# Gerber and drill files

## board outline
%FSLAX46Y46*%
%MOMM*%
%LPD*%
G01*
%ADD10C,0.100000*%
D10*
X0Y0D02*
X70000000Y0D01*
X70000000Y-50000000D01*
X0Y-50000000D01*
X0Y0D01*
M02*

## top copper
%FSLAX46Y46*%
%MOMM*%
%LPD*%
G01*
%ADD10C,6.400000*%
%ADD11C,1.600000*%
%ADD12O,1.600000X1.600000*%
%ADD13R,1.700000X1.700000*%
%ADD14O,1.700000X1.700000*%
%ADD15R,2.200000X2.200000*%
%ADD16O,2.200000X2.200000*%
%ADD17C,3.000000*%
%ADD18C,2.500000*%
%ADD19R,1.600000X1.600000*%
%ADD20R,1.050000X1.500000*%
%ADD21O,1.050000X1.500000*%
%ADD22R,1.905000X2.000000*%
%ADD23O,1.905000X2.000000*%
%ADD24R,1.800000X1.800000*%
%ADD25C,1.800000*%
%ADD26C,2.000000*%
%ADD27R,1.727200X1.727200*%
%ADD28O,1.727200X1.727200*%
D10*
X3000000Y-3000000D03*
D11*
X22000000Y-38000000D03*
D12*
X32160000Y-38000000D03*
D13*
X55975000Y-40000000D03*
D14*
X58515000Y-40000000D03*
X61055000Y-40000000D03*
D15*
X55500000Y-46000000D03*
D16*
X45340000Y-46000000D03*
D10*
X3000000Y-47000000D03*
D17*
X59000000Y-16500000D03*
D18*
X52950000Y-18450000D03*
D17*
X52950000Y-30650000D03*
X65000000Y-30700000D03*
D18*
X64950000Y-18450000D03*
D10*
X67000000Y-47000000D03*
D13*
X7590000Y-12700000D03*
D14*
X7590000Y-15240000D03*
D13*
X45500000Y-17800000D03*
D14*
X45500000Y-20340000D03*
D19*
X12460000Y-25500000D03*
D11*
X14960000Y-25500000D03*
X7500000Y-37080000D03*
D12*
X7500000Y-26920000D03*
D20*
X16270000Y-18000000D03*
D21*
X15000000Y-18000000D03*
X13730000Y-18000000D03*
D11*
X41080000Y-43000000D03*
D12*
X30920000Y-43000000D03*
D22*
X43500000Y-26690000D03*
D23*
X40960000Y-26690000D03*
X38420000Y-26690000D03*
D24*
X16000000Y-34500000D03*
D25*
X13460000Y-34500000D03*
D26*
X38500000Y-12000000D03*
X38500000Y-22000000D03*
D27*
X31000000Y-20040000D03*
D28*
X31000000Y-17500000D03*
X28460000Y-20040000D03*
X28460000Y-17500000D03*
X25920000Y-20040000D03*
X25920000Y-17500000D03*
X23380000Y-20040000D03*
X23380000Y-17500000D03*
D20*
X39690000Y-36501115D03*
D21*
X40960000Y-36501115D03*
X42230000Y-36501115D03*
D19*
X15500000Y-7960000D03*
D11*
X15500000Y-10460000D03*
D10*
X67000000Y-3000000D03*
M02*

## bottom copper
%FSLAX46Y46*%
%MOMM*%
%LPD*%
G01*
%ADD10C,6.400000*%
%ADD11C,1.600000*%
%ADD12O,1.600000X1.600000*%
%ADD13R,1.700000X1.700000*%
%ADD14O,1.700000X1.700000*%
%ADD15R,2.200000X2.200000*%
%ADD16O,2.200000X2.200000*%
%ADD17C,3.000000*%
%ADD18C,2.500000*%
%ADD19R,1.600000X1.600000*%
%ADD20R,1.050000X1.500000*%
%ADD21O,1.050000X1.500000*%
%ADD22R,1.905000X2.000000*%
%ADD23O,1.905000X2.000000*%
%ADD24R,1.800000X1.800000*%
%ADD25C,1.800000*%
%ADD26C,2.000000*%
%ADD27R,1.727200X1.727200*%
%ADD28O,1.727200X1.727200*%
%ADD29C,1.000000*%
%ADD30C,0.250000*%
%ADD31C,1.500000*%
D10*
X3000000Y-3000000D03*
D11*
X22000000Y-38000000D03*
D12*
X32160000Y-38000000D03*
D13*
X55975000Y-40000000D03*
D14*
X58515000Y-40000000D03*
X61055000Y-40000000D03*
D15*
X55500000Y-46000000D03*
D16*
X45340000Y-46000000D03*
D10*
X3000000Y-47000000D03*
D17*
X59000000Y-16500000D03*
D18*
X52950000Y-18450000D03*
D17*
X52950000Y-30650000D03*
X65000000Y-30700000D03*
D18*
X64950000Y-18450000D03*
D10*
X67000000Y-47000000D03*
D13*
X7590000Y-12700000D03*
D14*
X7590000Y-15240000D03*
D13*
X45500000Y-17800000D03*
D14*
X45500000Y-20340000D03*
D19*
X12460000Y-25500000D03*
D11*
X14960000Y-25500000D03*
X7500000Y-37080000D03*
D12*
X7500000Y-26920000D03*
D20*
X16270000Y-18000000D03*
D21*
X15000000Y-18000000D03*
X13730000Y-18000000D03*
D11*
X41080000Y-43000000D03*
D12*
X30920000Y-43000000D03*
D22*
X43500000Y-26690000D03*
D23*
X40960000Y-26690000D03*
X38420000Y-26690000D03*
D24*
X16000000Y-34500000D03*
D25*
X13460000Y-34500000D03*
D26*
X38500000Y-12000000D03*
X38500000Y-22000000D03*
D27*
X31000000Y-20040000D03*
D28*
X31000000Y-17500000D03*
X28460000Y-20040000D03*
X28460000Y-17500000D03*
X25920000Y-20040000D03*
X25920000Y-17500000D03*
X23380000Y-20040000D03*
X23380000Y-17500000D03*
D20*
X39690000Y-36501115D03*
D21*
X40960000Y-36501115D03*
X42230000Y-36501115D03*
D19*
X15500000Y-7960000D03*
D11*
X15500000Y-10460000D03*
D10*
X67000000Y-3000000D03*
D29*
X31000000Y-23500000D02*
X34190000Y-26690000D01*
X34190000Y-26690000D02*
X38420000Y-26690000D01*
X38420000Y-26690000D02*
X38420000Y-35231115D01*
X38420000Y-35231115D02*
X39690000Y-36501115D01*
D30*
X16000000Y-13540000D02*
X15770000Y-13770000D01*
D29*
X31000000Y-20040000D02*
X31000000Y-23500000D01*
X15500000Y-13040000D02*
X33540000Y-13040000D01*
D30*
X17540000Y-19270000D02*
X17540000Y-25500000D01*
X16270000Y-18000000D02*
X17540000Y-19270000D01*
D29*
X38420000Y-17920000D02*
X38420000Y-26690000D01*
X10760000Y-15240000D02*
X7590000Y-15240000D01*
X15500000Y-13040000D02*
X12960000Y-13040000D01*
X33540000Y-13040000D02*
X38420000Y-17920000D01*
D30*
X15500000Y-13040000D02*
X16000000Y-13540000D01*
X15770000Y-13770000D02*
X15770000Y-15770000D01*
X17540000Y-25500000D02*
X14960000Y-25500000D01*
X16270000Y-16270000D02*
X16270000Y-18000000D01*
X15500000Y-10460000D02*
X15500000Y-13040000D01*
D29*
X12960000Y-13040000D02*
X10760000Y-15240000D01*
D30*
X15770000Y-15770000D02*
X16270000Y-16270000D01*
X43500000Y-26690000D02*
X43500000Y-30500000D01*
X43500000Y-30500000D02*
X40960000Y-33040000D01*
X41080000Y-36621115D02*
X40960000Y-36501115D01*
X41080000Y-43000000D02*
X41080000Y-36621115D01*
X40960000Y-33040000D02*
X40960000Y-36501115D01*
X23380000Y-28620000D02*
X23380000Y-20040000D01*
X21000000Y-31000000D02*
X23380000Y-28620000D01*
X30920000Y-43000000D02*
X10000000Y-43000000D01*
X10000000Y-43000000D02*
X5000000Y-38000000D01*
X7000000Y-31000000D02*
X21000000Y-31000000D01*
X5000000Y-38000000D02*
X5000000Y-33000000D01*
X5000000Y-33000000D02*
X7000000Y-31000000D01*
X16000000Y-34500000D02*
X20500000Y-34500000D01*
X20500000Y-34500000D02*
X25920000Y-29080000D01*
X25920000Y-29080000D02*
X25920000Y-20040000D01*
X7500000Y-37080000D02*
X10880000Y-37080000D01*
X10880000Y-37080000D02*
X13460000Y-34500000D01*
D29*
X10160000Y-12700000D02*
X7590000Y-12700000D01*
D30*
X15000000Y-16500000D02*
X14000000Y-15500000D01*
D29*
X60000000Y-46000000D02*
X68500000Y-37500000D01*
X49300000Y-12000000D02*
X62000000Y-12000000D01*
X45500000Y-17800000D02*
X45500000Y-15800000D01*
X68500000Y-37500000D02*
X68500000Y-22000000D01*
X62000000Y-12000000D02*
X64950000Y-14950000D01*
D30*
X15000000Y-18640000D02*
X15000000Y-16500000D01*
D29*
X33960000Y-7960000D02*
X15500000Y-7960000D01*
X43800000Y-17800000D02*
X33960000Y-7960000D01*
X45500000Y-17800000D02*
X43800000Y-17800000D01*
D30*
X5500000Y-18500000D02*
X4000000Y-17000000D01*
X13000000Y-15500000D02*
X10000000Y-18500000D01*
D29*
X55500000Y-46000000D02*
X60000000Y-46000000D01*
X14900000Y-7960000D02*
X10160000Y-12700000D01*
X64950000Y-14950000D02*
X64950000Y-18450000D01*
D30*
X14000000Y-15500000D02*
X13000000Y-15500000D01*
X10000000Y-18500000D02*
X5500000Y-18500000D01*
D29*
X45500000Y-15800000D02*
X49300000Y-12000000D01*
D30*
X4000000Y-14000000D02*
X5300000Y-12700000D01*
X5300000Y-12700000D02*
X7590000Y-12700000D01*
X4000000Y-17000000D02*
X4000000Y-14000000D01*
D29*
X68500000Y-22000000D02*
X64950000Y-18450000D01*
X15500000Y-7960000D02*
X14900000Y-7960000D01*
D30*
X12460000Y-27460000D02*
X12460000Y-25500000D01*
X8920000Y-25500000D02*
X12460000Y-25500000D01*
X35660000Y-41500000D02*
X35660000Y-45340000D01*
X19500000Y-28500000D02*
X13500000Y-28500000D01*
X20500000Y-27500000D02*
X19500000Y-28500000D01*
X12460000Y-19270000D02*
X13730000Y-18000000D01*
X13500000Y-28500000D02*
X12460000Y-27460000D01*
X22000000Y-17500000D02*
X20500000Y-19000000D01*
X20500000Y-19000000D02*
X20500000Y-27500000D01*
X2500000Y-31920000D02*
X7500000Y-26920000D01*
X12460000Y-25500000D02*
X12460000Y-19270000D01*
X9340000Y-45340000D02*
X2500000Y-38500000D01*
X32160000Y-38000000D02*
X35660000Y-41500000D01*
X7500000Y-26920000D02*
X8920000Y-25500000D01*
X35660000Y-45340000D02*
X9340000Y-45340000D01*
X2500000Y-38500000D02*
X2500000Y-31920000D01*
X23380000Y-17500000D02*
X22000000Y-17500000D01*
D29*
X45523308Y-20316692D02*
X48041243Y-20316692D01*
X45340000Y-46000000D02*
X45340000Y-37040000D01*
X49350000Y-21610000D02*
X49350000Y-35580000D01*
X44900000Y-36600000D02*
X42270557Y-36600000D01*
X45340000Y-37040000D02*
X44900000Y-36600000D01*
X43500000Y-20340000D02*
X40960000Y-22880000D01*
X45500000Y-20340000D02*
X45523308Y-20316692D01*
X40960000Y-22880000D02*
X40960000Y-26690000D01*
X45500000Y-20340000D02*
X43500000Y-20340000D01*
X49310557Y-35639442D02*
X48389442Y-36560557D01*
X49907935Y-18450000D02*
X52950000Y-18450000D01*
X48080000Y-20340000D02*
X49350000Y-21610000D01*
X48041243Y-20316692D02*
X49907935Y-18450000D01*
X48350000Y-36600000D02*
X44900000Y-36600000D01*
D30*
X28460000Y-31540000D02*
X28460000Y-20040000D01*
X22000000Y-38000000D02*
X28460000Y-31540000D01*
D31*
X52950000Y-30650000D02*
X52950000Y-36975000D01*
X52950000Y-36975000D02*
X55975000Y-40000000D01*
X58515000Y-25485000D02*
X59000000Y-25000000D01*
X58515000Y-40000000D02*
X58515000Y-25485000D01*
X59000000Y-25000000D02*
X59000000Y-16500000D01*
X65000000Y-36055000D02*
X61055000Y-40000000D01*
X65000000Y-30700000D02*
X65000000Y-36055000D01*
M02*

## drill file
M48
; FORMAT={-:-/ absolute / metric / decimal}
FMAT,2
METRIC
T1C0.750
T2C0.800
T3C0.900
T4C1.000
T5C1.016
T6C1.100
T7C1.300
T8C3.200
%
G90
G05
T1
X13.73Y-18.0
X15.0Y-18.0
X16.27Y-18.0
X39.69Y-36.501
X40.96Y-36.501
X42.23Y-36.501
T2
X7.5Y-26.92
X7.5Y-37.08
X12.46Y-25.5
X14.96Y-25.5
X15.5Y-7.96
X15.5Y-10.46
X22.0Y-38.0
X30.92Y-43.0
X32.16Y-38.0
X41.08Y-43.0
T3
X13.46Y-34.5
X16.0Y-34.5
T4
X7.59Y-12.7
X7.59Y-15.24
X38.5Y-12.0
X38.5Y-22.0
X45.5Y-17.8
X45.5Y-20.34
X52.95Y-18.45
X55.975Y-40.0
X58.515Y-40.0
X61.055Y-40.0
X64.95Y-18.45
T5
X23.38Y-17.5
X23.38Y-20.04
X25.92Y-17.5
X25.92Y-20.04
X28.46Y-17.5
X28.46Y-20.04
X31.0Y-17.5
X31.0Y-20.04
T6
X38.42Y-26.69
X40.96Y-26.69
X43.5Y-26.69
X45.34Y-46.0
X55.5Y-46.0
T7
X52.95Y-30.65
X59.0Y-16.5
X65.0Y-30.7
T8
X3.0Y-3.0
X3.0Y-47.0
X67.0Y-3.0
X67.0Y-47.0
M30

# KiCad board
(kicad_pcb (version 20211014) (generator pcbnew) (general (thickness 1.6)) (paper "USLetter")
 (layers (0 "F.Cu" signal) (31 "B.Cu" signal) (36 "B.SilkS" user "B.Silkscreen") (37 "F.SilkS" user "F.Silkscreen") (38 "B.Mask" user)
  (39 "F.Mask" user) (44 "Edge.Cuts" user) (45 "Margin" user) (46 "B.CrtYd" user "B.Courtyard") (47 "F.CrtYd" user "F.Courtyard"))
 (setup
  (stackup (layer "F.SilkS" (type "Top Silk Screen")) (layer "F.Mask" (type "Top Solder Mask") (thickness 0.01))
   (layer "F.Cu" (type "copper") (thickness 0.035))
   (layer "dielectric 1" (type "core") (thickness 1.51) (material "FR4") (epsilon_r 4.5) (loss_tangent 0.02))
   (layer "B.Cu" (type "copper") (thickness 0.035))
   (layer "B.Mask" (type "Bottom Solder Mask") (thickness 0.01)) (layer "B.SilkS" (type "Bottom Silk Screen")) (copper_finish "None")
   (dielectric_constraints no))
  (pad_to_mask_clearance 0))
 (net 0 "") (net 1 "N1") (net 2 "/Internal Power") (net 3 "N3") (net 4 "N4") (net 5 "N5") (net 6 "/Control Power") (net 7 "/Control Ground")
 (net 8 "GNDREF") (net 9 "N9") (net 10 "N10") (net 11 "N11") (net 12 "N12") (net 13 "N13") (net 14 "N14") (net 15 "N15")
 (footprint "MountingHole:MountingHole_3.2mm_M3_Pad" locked (layer "F.Cu") (at 3 3)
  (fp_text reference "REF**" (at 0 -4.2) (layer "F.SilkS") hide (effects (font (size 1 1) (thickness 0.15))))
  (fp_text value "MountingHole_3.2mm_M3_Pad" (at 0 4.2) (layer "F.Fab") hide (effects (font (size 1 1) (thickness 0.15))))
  (pad "1" thru_hole circle locked (at 0 0) (size 6.4 6.4) (drill 3.2) (layers *.Cu *.Mask)))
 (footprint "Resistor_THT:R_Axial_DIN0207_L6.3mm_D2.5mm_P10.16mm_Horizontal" (layer "F.Cu") (at 22 38)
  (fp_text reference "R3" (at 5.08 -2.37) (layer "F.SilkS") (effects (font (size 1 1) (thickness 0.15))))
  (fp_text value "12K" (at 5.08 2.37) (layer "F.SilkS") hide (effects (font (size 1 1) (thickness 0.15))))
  (pad "1" thru_hole circle (at 0 0) (size 1.6 1.6) (drill 0.8) (layers *.Cu *.Mask) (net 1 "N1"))
  (pad "2" thru_hole oval (at 10.16 0) (size 1.6 1.6) (drill 0.8) (layers *.Cu *.Mask) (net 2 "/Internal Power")))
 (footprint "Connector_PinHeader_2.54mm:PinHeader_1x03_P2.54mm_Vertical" (layer "F.Cu") (at 55.975 40 90)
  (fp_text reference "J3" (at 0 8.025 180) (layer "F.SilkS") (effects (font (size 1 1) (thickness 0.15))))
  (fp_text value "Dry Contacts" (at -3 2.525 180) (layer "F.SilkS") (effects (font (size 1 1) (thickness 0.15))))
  (pad "1" thru_hole rect (at 0 0 90) (size 1.7 1.7) (drill 1) (layers *.Cu *.Mask) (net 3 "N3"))
  (pad "2" thru_hole oval (at 0 2.54 90) (size 1.7 1.7) (drill 1) (layers *.Cu *.Mask) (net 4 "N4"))
  (pad "3" thru_hole oval (at 0 5.08 90) (size 1.7 1.7) (drill 1) (layers *.Cu *.Mask) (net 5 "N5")))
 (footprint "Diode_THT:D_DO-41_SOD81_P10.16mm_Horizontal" (layer "F.Cu") (at 55.5 46 180)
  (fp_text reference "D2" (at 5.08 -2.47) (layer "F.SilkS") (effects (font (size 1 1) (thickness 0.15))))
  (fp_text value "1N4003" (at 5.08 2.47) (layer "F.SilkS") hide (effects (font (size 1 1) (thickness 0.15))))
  (pad "1" thru_hole rect (at 0 0 180) (size 2.2 2.2) (drill 1.1) (layers *.Cu *.Mask) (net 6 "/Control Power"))
  (pad "2" thru_hole oval (at 10.16 0 180) (size 2.2 2.2) (drill 1.1) (layers *.Cu *.Mask) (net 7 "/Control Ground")))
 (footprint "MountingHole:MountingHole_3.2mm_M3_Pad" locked (layer "F.Cu") (at 3 47)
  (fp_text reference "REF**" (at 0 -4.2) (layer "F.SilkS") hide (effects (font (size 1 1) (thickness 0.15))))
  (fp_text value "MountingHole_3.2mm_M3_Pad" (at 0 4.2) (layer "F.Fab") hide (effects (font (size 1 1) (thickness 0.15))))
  (pad "4" thru_hole circle locked (at 0 0) (size 6.4 6.4) (drill 3.2) (layers *.Cu *.Mask)))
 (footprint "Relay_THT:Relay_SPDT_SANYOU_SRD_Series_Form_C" (layer "F.Cu") (at 59 16.5 -90)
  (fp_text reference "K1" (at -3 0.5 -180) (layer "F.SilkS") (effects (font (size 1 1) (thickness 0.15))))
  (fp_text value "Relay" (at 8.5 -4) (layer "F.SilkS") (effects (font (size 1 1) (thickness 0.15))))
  (pad "1" thru_hole circle (at 0 0) (size 3 3) (drill 1.3) (layers *.Cu *.Mask) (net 4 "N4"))
  (pad "2" thru_hole circle (at 1.95 6.05) (size 2.5 2.5) (drill 1) (layers *.Cu *.Mask) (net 7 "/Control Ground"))
  (pad "3" thru_hole circle (at 14.15 6.05) (size 3 3) (drill 1.3) (layers *.Cu *.Mask) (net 3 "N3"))
  (pad "4" thru_hole circle (at 14.2 -6) (size 3 3) (drill 1.3) (layers *.Cu *.Mask) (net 5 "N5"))
  (pad "5" thru_hole circle (at 1.95 -5.95) (size 2.5 2.5) (drill 1) (layers *.Cu *.Mask) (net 6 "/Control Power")))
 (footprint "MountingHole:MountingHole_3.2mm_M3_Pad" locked (layer "F.Cu") (at 67 47)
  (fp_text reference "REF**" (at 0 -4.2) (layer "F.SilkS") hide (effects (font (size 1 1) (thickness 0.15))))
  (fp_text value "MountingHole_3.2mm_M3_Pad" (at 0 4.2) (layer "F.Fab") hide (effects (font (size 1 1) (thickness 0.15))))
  (pad "3" thru_hole circle locked (at 0 0) (size 6.4 6.4) (drill 3.2) (layers *.Cu *.Mask)))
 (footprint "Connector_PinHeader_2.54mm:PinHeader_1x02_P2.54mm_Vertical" (layer "F.Cu") (at 7.59 12.7)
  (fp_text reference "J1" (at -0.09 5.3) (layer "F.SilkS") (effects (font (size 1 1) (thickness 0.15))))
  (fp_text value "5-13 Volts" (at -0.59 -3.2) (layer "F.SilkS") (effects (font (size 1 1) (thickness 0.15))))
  (pad "1" thru_hole rect (at 0 0) (size 1.7 1.7) (drill 1) (layers *.Cu *.Mask) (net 6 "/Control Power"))
  (pad "2" thru_hole oval (at 0 2.54) (size 1.7 1.7) (drill 1) (layers *.Cu *.Mask) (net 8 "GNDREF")))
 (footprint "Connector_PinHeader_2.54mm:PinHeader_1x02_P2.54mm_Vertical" (layer "F.Cu") (at 45.5 17.8)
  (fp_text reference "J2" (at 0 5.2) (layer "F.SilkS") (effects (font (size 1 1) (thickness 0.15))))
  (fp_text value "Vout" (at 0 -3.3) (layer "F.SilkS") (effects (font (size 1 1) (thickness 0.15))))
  (pad "1" thru_hole rect (at 0 0) (size 1.7 1.7) (drill 1) (layers *.Cu *.Mask) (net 6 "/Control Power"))
  (pad "2" thru_hole oval (at 0 2.54) (size 1.7 1.7) (drill 1) (layers *.Cu *.Mask) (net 7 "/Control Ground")))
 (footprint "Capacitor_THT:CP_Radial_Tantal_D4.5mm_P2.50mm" (layer "F.Cu") (at 12.46 25.5)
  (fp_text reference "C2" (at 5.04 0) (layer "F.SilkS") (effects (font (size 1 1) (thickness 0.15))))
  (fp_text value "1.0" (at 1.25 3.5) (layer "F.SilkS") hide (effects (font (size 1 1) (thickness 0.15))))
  (pad "1" thru_hole rect (at 0 0) (size 1.6 1.6) (drill 0.8) (layers *.Cu *.Mask) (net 2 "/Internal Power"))
  (pad "2" thru_hole circle (at 2.5 0) (size 1.6 1.6) (drill 0.8) (layers *.Cu *.Mask) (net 8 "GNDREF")))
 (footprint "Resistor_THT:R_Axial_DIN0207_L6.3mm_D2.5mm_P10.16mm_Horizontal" (layer "F.Cu") (at 7.5 37.08 90)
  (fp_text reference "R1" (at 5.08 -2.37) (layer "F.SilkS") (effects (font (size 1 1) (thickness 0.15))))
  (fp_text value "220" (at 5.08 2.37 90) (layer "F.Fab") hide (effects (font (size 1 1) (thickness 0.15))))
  (pad "1" thru_hole circle (at 0 0 90) (size 1.6 1.6) (drill 0.8) (layers *.Cu *.Mask) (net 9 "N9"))
  (pad "2" thru_hole oval (at 10.16 0 90) (size 1.6 1.6) (drill 0.8) (layers *.Cu *.Mask) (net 2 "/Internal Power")))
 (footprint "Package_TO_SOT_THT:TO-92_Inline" (layer "F.Cu") (at 16.27 18 180)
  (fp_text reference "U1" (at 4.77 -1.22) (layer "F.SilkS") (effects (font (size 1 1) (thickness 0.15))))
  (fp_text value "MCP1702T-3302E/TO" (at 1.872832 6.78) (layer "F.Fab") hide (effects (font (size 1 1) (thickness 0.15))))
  (pad "1" thru_hole rect (at 0 0 180) (size 1.05 1.5) (drill 0.75) (layers *.Cu *.Mask) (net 8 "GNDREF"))
  (pad "2" thru_hole oval (at 1.27 0 180) (size 1.05 1.5) (drill 0.75) (layers *.Cu *.Mask) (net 6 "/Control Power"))
  (pad "3" thru_hole oval (at 2.54 0 180) (size 1.05 1.5) (drill 0.75) (layers *.Cu *.Mask) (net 2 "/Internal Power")))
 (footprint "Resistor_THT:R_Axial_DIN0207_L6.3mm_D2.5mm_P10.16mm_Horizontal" (layer "F.Cu") (at 41.08 43 180)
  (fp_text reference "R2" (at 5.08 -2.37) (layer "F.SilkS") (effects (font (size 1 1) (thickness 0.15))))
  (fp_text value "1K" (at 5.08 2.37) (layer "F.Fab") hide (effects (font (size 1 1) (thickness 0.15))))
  (pad "1" thru_hole circle (at 0 0 180) (size 1.6 1.6) (drill 0.8) (layers *.Cu *.Mask) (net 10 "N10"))
  (pad "2" thru_hole oval (at 10.16 0 180) (size 1.6 1.6) (drill 0.8) (layers *.Cu *.Mask) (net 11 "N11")))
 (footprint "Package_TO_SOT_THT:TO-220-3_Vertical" (layer "F.Cu") (at 43.5 26.69 180)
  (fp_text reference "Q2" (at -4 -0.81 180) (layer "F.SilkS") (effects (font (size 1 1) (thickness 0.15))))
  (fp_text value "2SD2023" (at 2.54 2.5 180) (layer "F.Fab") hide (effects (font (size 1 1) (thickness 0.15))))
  (pad "1" thru_hole rect (at 0 0 180) (size 1.905 2) (drill 1.1) (layers *.Cu *.Mask) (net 10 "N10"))
  (pad "2" thru_hole oval (at 2.54 0 180) (size 1.905 2) (drill 1.1) (layers *.Cu *.Mask) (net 7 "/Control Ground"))
  (pad "3" thru_hole oval (at 5.08 0 180) (size 1.905 2) (drill 1.1) (layers *.Cu *.Mask) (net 8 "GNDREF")))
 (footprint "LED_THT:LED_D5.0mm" (layer "F.Cu") (at 16 34.5 180)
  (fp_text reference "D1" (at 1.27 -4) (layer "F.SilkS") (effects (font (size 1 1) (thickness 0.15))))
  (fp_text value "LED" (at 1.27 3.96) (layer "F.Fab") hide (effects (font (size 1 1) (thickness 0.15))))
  (pad "1" thru_hole rect (at 0 0 180) (size 1.8 1.8) (drill 0.9) (layers *.Cu *.Mask) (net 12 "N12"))
  (pad "2" thru_hole circle (at 2.54 0 180) (size 1.8 1.8) (drill 0.9) (layers *.Cu *.Mask) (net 9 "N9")))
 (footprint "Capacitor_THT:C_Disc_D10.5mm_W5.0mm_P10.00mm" (layer "F.Cu") (at 38.5 12 -90)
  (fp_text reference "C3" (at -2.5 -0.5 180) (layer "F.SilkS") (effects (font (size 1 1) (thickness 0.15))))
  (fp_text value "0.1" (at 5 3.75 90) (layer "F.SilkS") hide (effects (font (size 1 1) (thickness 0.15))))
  (pad "1" thru_hole circle (at 0 0 270) (size 2 2) (drill 1) (layers *.Cu *.Mask) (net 6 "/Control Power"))
  (pad "2" thru_hole circle (at 10 0 270) (size 2 2) (drill 1) (layers *.Cu *.Mask) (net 8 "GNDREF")))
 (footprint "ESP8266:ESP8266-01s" (layer "F.Cu") (at 31 17.5 -90)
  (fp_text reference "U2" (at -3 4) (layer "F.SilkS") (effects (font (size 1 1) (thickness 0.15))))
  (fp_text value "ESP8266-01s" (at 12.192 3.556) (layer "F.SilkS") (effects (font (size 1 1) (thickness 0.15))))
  (pad "1" thru_hole rect (at 2.54 0 270) (size 1.7272 1.7272) (drill 1.016) (layers *.Cu *.Mask) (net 8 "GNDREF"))
  (pad "2" thru_hole oval (at 0 0 270) (size 1.7272 1.7272) (drill 1.016) (layers *.Cu *.Mask) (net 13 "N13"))
  (pad "3" thru_hole oval (at 2.54 2.54 270) (size 1.7272 1.7272) (drill 1.016) (layers *.Cu *.Mask) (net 1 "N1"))
  (pad "4" thru_hole oval (at 0 2.54 270) (size 1.7272 1.7272) (drill 1.016) (layers *.Cu *.Mask) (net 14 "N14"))
  (pad "5" thru_hole oval (at 2.54 5.08 270) (size 1.7272 1.7272) (drill 1.016) (layers *.Cu *.Mask) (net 12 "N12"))
  (pad "6" thru_hole oval (at 0 5.08 270) (size 1.7272 1.7272) (drill 1.016) (layers *.Cu *.Mask) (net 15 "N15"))
  (pad "7" thru_hole oval (at 2.54 7.62 270) (size 1.7272 1.7272) (drill 1.016) (layers *.Cu *.Mask) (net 11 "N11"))
  (pad "8" thru_hole oval (at 0 7.62 270) (size 1.7272 1.7272) (drill 1.016) (layers *.Cu *.Mask) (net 2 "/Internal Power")))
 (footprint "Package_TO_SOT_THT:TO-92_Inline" (layer "F.Cu") (at 39.69 36.501115)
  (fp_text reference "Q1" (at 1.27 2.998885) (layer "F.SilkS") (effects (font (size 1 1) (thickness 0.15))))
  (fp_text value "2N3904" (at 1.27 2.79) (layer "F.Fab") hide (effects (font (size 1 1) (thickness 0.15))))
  (pad "1" thru_hole rect (at 0 0) (size 1.05 1.5) (drill 0.75) (layers *.Cu *.Mask) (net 8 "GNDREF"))
  (pad "2" thru_hole oval (at 1.27 0) (size 1.05 1.5) (drill 0.75) (layers *.Cu *.Mask) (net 10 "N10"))
  (pad "3" thru_hole oval (at 2.54 0) (size 1.05 1.5) (drill 0.75) (layers *.Cu *.Mask) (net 7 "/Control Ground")))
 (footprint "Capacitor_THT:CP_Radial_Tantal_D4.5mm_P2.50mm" (layer "F.Cu") (at 15.5 7.96 -90)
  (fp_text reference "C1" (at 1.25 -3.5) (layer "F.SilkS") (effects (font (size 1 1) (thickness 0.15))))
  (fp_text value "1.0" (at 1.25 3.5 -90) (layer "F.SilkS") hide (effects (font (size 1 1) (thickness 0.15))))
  (pad "1" thru_hole rect (at 0 0 270) (size 1.6 1.6) (drill 0.8) (layers *.Cu *.Mask) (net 6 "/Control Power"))
  (pad "2" thru_hole circle (at 2.5 0 270) (size 1.6 1.6) (drill 0.8) (layers *.Cu *.Mask) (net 8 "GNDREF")))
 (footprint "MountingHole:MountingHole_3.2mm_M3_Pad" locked (layer "F.Cu") (at 67 3)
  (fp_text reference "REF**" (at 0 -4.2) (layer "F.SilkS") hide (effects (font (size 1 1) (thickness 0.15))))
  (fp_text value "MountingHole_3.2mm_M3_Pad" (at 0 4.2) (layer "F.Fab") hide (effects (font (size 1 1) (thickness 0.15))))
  (pad "2" thru_hole circle locked (at 0 0) (size 6.4 6.4) (drill 3.2) (layers *.Cu *.Mask)))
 (gr_rect locked (start 0 0) (end 70 50) (layer "Edge.Cuts") (width 0.1) (fill none))
 (segment (start 31 23.5) (end 34.19 26.69) (width 1) (layer "B.Cu") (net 8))
 (segment (start 34.19 26.69) (end 38.42 26.69) (width 1) (layer "B.Cu") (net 8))
 (segment (start 38.42 26.69) (end 38.42 35.231115) (width 1) (layer "B.Cu") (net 8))
 (segment (start 38.42 35.231115) (end 39.69 36.501115) (width 1) (layer "B.Cu") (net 8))
 (segment (start 16 13.54) (end 15.77 13.77) (width 0.25) (layer "B.Cu") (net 8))
 (segment (start 31 20.04) (end 31 23.5) (width 1) (layer "B.Cu") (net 8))
 (segment (start 15.5 13.04) (end 33.54 13.04) (width 1) (layer "B.Cu") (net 8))
 (segment (start 17.54 19.27) (end 17.54 25.5) (width 0.25) (layer "B.Cu") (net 8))
 (segment (start 16.27 18) (end 17.54 19.27) (width 0.25) (layer "B.Cu") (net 8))
 (segment (start 38.42 17.92) (end 38.42 26.69) (width 1) (layer "B.Cu") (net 8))
 (segment (start 10.76 15.24) (end 7.59 15.24) (width 1) (layer "B.Cu") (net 8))
 (segment (start 15.5 13.04) (end 12.96 13.04) (width 1) (layer "B.Cu") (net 8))
 (segment (start 33.54 13.04) (end 38.42 17.92) (width 1) (layer "B.Cu") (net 8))
 (segment (start 15.5 13.04) (end 16 13.54) (width 0.25) (layer "B.Cu") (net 8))
 (segment (start 15.77 13.77) (end 15.77 15.77) (width 0.25) (layer "B.Cu") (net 8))
 (segment (start 17.54 25.5) (end 14.96 25.5) (width 0.25) (layer "B.Cu") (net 8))
 (segment (start 16.27 16.27) (end 16.27 18) (width 0.25) (layer "B.Cu") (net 8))
 (segment (start 15.5 10.46) (end 15.5 13.04) (width 0.25) (layer "B.Cu") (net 8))
 (segment (start 12.96 13.04) (end 10.76 15.24) (width 1) (layer "B.Cu") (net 8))
 (segment (start 15.77 15.77) (end 16.27 16.27) (width 0.25) (layer "B.Cu") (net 8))
 (segment (start 43.5 26.69) (end 43.5 30.5) (width 0.25) (layer "B.Cu") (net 10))
 (segment (start 43.5 30.5) (end 40.96 33.04) (width 0.25) (layer "B.Cu") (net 10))
 (segment (start 41.08 36.621115) (end 40.96 36.501115) (width 0.25) (layer "B.Cu") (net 10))
 (segment (start 41.08 43) (end 41.08 36.621115) (width 0.25) (layer "B.Cu") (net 10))
 (segment (start 40.96 33.04) (end 40.96 36.501115) (width 0.25) (layer "B.Cu") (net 10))
 (segment (start 23.38 28.62) (end 23.38 20.04) (width 0.25) (layer "B.Cu") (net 11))
 (segment (start 21 31) (end 23.38 28.62) (width 0.25) (layer "B.Cu") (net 11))
 (segment (start 30.92 43) (end 10 43) (width 0.25) (layer "B.Cu") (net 11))
 (segment (start 10 43) (end 5 38) (width 0.25) (layer "B.Cu") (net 11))
 (segment (start 7 31) (end 21 31) (width 0.25) (layer "B.Cu") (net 11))
 (segment (start 5 38) (end 5 33) (width 0.25) (layer "B.Cu") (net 11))
 (segment (start 5 33) (end 7 31) (width 0.25) (layer "B.Cu") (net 11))
 (segment (start 16 34.5) (end 20.5 34.5) (width 0.25) (layer "B.Cu") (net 12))
 (segment (start 20.5 34.5) (end 25.92 29.08) (width 0.25) (layer "B.Cu") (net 12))
 (segment (start 25.92 29.08) (end 25.92 20.04) (width 0.25) (layer "B.Cu") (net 12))
 (segment (start 7.5 37.08) (end 10.88 37.08) (width 0.25) (layer "B.Cu") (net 9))
 (segment (start 10.88 37.08) (end 13.46 34.5) (width 0.25) (layer "B.Cu") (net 9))
 (segment (start 10.16 12.7) (end 7.59 12.7) (width 1) (layer "B.Cu") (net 6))
 (segment (start 15 16.5) (end 14 15.5) (width 0.25) (layer "B.Cu") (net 6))
 (segment (start 60 46) (end 68.5 37.5) (width 1) (layer "B.Cu") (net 6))
 (segment (start 49.3 12) (end 62 12) (width 1) (layer "B.Cu") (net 6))
 (segment (start 45.5 17.8) (end 45.5 15.8) (width 1) (layer "B.Cu") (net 6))
 (segment (start 68.5 37.5) (end 68.5 22) (width 1) (layer "B.Cu") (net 6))
 (segment (start 62 12) (end 64.95 14.95) (width 1) (layer "B.Cu") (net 6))
 (segment (start 15 18.64) (end 15 16.5) (width 0.25) (layer "B.Cu") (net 6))
 (segment (start 33.96 7.96) (end 15.5 7.96) (width 1) (layer "B.Cu") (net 6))
 (segment (start 43.8 17.8) (end 33.96 7.96) (width 1) (layer "B.Cu") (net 6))
 (segment (start 45.5 17.8) (end 43.8 17.8) (width 1) (layer "B.Cu") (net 6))
 (segment (start 5.5 18.5) (end 4 17) (width 0.25) (layer "B.Cu") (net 6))
 (segment (start 13 15.5) (end 10 18.5) (width 0.25) (layer "B.Cu") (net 6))
 (segment (start 55.5 46) (end 60 46) (width 1) (layer "B.Cu") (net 6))
 (segment (start 14.9 7.96) (end 10.16 12.7) (width 1) (layer "B.Cu") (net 6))
 (segment (start 64.95 14.95) (end 64.95 18.45) (width 1) (layer "B.Cu") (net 6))
 (segment (start 14 15.5) (end 13 15.5) (width 0.25) (layer "B.Cu") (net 6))
 (segment (start 10 18.5) (end 5.5 18.5) (width 0.25) (layer "B.Cu") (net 6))
 (segment (start 45.5 15.8) (end 49.3 12) (width 1) (layer "B.Cu") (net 6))
 (segment (start 4 14) (end 5.3 12.7) (width 0.25) (layer "B.Cu") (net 6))
 (segment (start 5.3 12.7) (end 7.59 12.7) (width 0.25) (layer "B.Cu") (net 6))
 (segment (start 4 17) (end 4 14) (width 0.25) (layer "B.Cu") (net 6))
 (segment (start 68.5 22) (end 64.95 18.45) (width 1) (layer "B.Cu") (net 6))
 (segment (start 15.5 7.96) (end 14.9 7.96) (width 1) (layer "B.Cu") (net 6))
 (segment (start 12.46 27.46) (end 12.46 25.5) (width 0.25) (layer "B.Cu") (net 2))
 (segment (start 8.92 25.5) (end 12.46 25.5) (width 0.25) (layer "B.Cu") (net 2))
 (segment (start 35.66 41.5) (end 35.66 45.34) (width 0.25) (layer "B.Cu") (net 2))
 (segment (start 19.5 28.5) (end 13.5 28.5) (width 0.25) (layer "B.Cu") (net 2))
 (segment (start 20.5 27.5) (end 19.5 28.5) (width 0.25) (layer "B.Cu") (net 2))
 (segment (start 12.46 19.27) (end 13.73 18) (width 0.25) (layer "B.Cu") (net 2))
 (segment (start 13.5 28.5) (end 12.46 27.46) (width 0.25) (layer "B.Cu") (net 2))
 (segment (start 22 17.5) (end 20.5 19) (width 0.25) (layer "B.Cu") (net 2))
 (segment (start 20.5 19) (end 20.5 27.5) (width 0.25) (layer "B.Cu") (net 2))
 (segment (start 2.5 31.92) (end 7.5 26.92) (width 0.25) (layer "B.Cu") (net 2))
 (segment (start 12.46 25.5) (end 12.46 19.27) (width 0.25) (layer "B.Cu") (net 2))
 (segment (start 9.34 45.34) (end 2.5 38.5) (width 0.25) (layer "B.Cu") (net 2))
 (segment (start 32.16 38) (end 35.66 41.5) (width 0.25) (layer "B.Cu") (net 2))
 (segment (start 7.5 26.92) (end 8.92 25.5) (width 0.25) (layer "B.Cu") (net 2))
 (segment (start 35.66 45.34) (end 9.34 45.34) (width 0.25) (layer "B.Cu") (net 2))
 (segment (start 2.5 38.5) (end 2.5 31.92) (width 0.25) (layer "B.Cu") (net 2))
 (segment (start 23.38 17.5) (end 22 17.5) (width 0.25) (layer "B.Cu") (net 2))
 (segment (start 45.523308 20.316692) (end 48.041243 20.316692) (width 1) (layer "B.Cu") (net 7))
 (segment (start 45.34 46) (end 45.34 37.04) (width 1) (layer "B.Cu") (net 7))
 (segment (start 49.35 21.61) (end 49.35 35.58) (width 1) (layer "B.Cu") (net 7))
 (segment (start 44.9 36.6) (end 42.270557 36.6) (width 1) (layer "B.Cu") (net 7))
 (segment (start 45.34 37.04) (end 44.9 36.6) (width 1) (layer "B.Cu") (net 7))
 (segment (start 43.5 20.34) (end 40.96 22.88) (width 1) (layer "B.Cu") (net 7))
 (segment (start 45.5 20.34) (end 45.523308 20.316692) (width 1) (layer "B.Cu") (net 7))
 (segment (start 40.96 22.88) (end 40.96 26.69) (width 1) (layer "B.Cu") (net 7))
 (segment (start 45.5 20.34) (end 43.5 20.34) (width 1) (layer "B.Cu") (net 7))
 (segment (start 49.310557 35.639442) (end 48.389442 36.560557) (width 1) (layer "B.Cu") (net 7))
 (segment (start 49.907935 18.45) (end 52.95 18.45) (width 1) (layer "B.Cu") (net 7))
 (segment (start 48.08 20.34) (end 49.35 21.61) (width 1) (layer "B.Cu") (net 7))
 (segment (start 48.041243 20.316692) (end 49.907935 18.45) (width 1) (layer "B.Cu") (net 7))
 (segment (start 48.35 36.6) (end 44.9 36.6) (width 1) (layer "B.Cu") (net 7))
 (segment (start 28.46 31.54) (end 28.46 20.04) (width 0.25) (layer "B.Cu") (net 1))
 (segment (start 22 38) (end 28.46 31.54) (width 0.25) (layer "B.Cu") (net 1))
 (segment (start 52.95 30.65) (end 52.95 36.975) (width 1.5) (layer "B.Cu") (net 3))
 (segment (start 52.95 36.975) (end 55.975 40) (width 1.5) (layer "B.Cu") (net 3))
 (segment (start 58.515 25.485) (end 59 25) (width 1.5) (layer "B.Cu") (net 4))
 (segment (start 58.515 40) (end 58.515 25.485) (width 1.5) (layer "B.Cu") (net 4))
 (segment (start 59 25) (end 59 16.5) (width 1.5) (layer "B.Cu") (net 4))
 (segment (start 65 36.055) (end 61.055 40) (width 1.5) (layer "B.Cu") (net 5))
 (segment (start 65 30.7) (end 65 36.055) (width 1.5) (layer "B.Cu") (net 5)))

